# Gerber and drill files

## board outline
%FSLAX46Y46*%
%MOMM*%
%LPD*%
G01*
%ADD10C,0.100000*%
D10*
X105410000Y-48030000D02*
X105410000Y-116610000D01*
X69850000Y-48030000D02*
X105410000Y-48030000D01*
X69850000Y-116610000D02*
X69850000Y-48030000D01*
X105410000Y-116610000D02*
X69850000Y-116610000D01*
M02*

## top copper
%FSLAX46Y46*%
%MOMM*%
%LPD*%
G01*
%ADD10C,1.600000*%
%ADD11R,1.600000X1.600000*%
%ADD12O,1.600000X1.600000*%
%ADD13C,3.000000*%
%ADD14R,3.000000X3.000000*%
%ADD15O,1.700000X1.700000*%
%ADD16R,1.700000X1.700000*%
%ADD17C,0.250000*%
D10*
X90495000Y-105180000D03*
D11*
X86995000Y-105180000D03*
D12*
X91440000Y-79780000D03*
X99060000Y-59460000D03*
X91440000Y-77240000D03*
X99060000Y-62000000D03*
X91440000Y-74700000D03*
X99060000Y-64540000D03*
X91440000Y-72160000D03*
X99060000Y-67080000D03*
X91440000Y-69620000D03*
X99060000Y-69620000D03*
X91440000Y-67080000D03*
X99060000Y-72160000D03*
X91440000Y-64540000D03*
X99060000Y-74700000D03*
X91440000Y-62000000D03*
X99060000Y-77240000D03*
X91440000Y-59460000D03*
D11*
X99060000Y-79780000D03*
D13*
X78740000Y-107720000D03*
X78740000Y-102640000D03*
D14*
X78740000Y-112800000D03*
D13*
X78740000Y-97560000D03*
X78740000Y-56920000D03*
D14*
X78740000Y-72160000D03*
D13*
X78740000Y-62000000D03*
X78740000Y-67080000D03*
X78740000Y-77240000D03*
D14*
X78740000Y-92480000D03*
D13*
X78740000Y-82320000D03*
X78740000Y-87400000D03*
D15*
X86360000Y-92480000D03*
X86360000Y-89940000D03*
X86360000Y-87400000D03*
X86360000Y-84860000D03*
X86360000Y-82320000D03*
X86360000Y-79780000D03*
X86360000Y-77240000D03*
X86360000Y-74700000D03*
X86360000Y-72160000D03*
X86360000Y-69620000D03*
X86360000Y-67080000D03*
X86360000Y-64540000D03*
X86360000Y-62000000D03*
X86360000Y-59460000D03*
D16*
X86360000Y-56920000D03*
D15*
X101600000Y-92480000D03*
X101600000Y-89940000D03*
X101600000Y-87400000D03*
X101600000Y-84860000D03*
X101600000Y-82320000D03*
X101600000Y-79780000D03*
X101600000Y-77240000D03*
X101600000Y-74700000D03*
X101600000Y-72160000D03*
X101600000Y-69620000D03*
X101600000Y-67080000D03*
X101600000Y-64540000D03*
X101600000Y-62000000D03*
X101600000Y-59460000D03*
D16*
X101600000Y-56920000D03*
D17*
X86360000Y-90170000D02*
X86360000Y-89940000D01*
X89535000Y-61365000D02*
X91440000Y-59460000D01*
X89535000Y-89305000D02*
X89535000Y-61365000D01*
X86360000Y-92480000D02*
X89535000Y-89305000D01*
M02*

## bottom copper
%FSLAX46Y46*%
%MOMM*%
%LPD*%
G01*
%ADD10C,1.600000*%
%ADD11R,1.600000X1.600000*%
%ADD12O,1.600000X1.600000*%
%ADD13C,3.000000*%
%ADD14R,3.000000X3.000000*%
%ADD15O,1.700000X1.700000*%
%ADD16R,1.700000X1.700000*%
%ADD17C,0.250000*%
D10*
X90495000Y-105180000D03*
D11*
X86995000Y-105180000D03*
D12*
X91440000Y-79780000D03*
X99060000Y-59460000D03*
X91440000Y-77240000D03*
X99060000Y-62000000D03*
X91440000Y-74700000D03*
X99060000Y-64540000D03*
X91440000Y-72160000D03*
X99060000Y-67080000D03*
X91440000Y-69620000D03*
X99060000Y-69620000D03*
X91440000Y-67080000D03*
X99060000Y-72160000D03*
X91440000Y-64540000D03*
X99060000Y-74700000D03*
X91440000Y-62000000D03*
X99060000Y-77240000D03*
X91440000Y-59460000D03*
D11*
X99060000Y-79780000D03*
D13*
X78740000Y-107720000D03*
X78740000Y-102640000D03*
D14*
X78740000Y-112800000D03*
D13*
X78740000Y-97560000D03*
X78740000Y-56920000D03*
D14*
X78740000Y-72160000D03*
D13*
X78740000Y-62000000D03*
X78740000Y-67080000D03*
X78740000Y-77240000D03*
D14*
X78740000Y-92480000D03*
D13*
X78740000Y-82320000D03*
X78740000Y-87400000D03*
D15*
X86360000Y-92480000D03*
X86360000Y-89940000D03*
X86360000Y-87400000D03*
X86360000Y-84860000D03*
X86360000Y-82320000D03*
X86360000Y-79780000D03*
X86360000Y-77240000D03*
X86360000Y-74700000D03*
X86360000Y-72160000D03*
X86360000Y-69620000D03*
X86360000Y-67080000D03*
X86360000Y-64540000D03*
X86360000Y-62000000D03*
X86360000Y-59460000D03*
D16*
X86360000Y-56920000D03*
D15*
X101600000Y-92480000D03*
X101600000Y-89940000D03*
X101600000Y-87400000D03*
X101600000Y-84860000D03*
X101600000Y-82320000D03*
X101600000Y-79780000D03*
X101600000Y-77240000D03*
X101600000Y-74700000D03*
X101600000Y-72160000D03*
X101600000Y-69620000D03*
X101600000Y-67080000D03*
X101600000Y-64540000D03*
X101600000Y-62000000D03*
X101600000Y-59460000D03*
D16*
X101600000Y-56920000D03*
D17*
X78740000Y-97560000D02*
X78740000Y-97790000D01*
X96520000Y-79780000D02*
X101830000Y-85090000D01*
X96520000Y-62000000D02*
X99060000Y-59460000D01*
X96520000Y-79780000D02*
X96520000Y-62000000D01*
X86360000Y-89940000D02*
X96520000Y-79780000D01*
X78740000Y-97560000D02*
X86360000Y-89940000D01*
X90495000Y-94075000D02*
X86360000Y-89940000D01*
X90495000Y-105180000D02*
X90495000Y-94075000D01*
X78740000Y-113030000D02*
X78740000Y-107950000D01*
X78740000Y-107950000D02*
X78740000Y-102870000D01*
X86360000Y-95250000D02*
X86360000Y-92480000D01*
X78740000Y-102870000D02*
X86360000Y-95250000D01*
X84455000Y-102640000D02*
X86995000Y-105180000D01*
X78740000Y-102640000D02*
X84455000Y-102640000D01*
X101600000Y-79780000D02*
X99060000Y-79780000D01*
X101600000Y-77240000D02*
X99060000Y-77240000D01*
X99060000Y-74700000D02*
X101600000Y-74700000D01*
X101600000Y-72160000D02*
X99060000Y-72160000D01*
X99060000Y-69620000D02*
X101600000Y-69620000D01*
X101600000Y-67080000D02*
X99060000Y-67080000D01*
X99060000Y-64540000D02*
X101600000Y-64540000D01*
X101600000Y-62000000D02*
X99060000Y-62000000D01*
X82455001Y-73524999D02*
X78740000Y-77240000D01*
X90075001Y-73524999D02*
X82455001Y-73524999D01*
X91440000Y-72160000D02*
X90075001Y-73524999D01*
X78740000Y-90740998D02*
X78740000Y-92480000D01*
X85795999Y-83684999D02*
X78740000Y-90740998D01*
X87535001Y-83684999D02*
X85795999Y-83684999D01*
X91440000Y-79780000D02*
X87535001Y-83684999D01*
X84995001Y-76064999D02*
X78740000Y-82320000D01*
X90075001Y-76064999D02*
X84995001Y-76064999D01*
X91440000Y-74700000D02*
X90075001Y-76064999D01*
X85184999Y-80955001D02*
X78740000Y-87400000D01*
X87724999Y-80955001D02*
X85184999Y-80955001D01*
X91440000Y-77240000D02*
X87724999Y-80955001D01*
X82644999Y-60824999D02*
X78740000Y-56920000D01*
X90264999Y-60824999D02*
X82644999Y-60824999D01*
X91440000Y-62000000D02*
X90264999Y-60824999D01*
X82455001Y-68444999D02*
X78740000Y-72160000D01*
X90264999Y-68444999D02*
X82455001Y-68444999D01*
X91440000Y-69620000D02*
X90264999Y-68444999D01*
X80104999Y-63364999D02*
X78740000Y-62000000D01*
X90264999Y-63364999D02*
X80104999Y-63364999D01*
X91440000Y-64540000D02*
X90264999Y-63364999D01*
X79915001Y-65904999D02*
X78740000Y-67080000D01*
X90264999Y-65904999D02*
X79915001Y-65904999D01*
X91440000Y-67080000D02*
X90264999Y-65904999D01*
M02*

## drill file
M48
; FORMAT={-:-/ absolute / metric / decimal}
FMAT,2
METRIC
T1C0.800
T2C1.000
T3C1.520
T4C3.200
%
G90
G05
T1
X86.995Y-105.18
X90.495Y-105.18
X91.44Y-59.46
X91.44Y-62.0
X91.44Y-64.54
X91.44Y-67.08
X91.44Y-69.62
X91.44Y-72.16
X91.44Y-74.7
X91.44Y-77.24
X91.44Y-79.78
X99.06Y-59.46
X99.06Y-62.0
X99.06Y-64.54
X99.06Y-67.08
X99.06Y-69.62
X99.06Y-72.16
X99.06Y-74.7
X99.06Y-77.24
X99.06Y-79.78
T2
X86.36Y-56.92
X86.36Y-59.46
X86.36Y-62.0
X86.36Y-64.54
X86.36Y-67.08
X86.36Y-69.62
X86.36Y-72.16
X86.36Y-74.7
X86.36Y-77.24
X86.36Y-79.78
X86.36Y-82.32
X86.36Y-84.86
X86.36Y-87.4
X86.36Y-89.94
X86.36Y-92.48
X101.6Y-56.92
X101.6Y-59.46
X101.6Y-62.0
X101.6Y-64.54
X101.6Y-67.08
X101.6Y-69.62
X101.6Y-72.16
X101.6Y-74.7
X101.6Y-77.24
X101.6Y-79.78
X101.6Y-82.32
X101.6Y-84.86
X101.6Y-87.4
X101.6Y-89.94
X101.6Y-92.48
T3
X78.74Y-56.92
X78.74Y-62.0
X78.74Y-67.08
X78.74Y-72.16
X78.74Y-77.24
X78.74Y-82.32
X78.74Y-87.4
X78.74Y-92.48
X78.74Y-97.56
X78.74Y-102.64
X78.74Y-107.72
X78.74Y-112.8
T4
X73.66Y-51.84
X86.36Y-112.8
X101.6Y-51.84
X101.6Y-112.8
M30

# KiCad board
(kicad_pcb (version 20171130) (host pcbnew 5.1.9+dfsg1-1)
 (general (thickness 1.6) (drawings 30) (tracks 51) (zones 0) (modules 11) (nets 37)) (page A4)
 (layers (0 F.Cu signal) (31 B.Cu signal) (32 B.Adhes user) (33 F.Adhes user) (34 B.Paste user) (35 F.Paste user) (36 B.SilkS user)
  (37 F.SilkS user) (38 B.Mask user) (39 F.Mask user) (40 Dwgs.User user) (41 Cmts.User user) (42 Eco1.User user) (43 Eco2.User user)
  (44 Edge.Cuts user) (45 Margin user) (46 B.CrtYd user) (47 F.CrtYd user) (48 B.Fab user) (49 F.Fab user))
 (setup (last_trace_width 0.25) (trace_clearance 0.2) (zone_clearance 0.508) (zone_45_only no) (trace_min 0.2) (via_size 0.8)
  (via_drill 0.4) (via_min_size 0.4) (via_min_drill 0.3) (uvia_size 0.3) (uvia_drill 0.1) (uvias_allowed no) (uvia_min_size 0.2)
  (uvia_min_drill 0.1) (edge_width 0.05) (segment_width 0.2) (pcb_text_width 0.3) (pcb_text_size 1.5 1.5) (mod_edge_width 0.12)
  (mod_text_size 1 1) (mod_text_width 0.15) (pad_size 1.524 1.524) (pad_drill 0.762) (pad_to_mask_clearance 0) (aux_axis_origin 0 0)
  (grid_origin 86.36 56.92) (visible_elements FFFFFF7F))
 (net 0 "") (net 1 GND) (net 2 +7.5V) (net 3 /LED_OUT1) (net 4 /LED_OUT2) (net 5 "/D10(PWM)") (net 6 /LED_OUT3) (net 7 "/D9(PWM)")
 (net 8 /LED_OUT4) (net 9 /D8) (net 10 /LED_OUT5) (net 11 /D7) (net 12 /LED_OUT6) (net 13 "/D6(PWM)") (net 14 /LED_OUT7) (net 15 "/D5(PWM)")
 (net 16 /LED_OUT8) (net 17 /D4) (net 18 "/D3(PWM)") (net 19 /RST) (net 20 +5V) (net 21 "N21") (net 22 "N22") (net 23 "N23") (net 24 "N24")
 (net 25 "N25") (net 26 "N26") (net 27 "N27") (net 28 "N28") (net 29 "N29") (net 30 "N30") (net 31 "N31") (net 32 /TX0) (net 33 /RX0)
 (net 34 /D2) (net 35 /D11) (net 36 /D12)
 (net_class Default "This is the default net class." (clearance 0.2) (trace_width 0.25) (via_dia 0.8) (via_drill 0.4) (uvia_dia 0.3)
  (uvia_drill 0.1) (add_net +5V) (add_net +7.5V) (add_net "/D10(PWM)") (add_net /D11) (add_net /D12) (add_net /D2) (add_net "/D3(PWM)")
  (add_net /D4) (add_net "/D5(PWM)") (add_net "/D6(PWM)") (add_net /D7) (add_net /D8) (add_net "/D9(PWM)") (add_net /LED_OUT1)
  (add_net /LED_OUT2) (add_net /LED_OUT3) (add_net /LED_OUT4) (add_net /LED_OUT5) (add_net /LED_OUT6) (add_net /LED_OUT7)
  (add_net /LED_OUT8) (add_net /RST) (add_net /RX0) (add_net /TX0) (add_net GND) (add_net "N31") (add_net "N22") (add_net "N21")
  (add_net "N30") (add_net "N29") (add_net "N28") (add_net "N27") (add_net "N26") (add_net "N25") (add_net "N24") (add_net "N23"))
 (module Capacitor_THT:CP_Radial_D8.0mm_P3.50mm (layer F.Cu) (at 86.995 105.18)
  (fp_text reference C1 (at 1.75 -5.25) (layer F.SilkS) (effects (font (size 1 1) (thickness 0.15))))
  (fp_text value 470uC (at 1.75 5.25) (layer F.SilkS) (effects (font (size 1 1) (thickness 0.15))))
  (pad 2 thru_hole circle (at 3.5 0) (size 1.6 1.6) (drill 0.8) (layers *.Cu *.Mask) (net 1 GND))
  (pad 1 thru_hole rect (at 0 0) (size 1.6 1.6) (drill 0.8) (layers *.Cu *.Mask) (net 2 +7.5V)))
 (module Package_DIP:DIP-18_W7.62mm (layer F.Cu) (at 99.06 79.78 180)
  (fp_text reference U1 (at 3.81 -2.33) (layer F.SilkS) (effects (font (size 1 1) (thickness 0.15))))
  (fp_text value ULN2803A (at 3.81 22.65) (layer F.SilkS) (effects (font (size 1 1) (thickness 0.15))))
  (pad 18 thru_hole oval (at 7.62 0 180) (size 1.6 1.6) (drill 0.8) (layers *.Cu *.Mask) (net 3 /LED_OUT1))
  (pad 9 thru_hole oval (at 0 20.32 180) (size 1.6 1.6) (drill 0.8) (layers *.Cu *.Mask) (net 1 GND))
  (pad 17 thru_hole oval (at 7.62 2.54 180) (size 1.6 1.6) (drill 0.8) (layers *.Cu *.Mask) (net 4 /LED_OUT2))
  (pad 8 thru_hole oval (at 0 17.78 180) (size 1.6 1.6) (drill 0.8) (layers *.Cu *.Mask) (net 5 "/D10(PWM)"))
  (pad 16 thru_hole oval (at 7.62 5.08 180) (size 1.6 1.6) (drill 0.8) (layers *.Cu *.Mask) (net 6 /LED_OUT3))
  (pad 7 thru_hole oval (at 0 15.24 180) (size 1.6 1.6) (drill 0.8) (layers *.Cu *.Mask) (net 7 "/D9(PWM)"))
  (pad 15 thru_hole oval (at 7.62 7.62 180) (size 1.6 1.6) (drill 0.8) (layers *.Cu *.Mask) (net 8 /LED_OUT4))
  (pad 6 thru_hole oval (at 0 12.7 180) (size 1.6 1.6) (drill 0.8) (layers *.Cu *.Mask) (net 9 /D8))
  (pad 14 thru_hole oval (at 7.62 10.16 180) (size 1.6 1.6) (drill 0.8) (layers *.Cu *.Mask) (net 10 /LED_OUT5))
  (pad 5 thru_hole oval (at 0 10.16 180) (size 1.6 1.6) (drill 0.8) (layers *.Cu *.Mask) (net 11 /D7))
  (pad 13 thru_hole oval (at 7.62 12.7 180) (size 1.6 1.6) (drill 0.8) (layers *.Cu *.Mask) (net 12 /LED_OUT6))
  (pad 4 thru_hole oval (at 0 7.62 180) (size 1.6 1.6) (drill 0.8) (layers *.Cu *.Mask) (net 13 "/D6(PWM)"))
  (pad 12 thru_hole oval (at 7.62 15.24 180) (size 1.6 1.6) (drill 0.8) (layers *.Cu *.Mask) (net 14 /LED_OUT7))
  (pad 3 thru_hole oval (at 0 5.08 180) (size 1.6 1.6) (drill 0.8) (layers *.Cu *.Mask) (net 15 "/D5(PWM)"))
  (pad 11 thru_hole oval (at 7.62 17.78 180) (size 1.6 1.6) (drill 0.8) (layers *.Cu *.Mask) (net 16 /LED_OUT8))
  (pad 2 thru_hole oval (at 0 2.54 180) (size 1.6 1.6) (drill 0.8) (layers *.Cu *.Mask) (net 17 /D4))
  (pad 10 thru_hole oval (at 7.62 20.32 180) (size 1.6 1.6) (drill 0.8) (layers *.Cu *.Mask) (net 2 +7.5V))
  (pad 1 thru_hole rect (at 0 0 180) (size 1.6 1.6) (drill 0.8) (layers *.Cu *.Mask) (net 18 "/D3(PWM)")))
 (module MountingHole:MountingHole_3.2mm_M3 (layer F.Cu) (at 101.6 51.84)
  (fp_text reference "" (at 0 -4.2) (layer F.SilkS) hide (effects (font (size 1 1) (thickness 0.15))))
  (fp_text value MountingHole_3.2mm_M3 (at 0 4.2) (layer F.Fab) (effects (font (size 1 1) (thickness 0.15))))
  (pad 1 np_thru_hole circle (at 0 0) (size 3.2 3.2) (drill 3.2) (layers *.Cu *.Mask)))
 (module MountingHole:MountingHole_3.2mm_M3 (layer F.Cu) (at 73.66 51.84)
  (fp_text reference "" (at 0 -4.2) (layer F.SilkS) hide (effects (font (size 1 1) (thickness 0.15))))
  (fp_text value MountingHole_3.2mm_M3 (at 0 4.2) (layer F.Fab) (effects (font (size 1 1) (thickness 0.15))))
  (pad 1 np_thru_hole circle (at 0 0) (size 3.2 3.2) (drill 3.2) (layers *.Cu *.Mask)))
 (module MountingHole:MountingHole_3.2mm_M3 (layer F.Cu) (at 101.6 112.8)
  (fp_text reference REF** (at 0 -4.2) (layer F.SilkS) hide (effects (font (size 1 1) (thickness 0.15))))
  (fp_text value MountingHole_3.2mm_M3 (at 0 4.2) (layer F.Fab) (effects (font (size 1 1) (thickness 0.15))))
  (pad 1 np_thru_hole circle (at 0 0) (size 3.2 3.2) (drill 3.2) (layers *.Cu *.Mask)))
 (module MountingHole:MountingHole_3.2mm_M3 (layer F.Cu) (at 86.36 112.8)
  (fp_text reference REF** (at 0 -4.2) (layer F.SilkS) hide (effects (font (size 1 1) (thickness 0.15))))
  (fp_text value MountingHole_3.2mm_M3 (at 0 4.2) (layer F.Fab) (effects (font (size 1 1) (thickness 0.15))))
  (pad 1 np_thru_hole circle (at 0 0) (size 3.2 3.2) (drill 3.2) (layers *.Cu *.Mask)))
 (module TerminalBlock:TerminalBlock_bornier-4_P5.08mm (layer F.Cu) (at 78.74 112.8 90)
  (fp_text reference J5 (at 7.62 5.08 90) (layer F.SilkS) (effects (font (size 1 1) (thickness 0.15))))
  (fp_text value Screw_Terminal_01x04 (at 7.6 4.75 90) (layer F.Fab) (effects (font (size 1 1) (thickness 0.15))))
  (pad 2 thru_hole circle (at 5.08 0 90) (size 3 3) (drill 1.52) (layers *.Cu *.Mask) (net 2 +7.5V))
  (pad 3 thru_hole circle (at 10.16 0 90) (size 3 3) (drill 1.52) (layers *.Cu *.Mask) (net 2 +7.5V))
  (pad 1 thru_hole rect (at 0 0 90) (size 3 3) (drill 1.52) (layers *.Cu *.Mask) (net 2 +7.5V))
  (pad 4 thru_hole circle (at 15.24 0 90) (size 3 3) (drill 1.52) (layers *.Cu *.Mask) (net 1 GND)))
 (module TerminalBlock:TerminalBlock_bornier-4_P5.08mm (layer F.Cu) (at 78.74 72.16 90)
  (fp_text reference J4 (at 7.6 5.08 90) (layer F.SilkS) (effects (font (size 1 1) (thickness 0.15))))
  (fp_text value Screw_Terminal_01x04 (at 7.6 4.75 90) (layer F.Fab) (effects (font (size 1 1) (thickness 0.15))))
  (pad 4 thru_hole circle (at 15.24 0 90) (size 3 3) (drill 1.52) (layers *.Cu *.Mask) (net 16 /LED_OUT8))
  (pad 1 thru_hole rect (at 0 0 90) (size 3 3) (drill 1.52) (layers *.Cu *.Mask) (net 10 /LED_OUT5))
  (pad 3 thru_hole circle (at 10.16 0 90) (size 3 3) (drill 1.52) (layers *.Cu *.Mask) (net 14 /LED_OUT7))
  (pad 2 thru_hole circle (at 5.08 0 90) (size 3 3) (drill 1.52) (layers *.Cu *.Mask) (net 12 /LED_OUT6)))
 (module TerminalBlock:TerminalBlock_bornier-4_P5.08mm (layer F.Cu) (at 78.74 92.48 90)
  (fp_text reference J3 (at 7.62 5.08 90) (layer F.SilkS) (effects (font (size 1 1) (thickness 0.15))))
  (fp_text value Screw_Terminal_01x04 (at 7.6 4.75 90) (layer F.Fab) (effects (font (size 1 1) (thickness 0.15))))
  (pad 4 thru_hole circle (at 15.24 0 90) (size 3 3) (drill 1.52) (layers *.Cu *.Mask) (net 8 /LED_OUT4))
  (pad 1 thru_hole rect (at 0 0 90) (size 3 3) (drill 1.52) (layers *.Cu *.Mask) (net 3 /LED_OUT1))
  (pad 3 thru_hole circle (at 10.16 0 90) (size 3 3) (drill 1.52) (layers *.Cu *.Mask) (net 6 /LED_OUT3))
  (pad 2 thru_hole circle (at 5.08 0 90) (size 3 3) (drill 1.52) (layers *.Cu *.Mask) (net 4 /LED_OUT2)))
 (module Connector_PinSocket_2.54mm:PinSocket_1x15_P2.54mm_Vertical (layer F.Cu) (at 86.36 56.92)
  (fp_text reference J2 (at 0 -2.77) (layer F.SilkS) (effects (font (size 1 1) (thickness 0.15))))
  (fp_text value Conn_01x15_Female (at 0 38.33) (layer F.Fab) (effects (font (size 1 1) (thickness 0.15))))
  (pad 15 thru_hole oval (at 0 35.56) (size 1.7 1.7) (drill 1) (layers *.Cu *.Mask) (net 2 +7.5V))
  (pad 14 thru_hole oval (at 0 33.02) (size 1.7 1.7) (drill 1) (layers *.Cu *.Mask) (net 1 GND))
  (pad 13 thru_hole oval (at 0 30.48) (size 1.7 1.7) (drill 1) (layers *.Cu *.Mask) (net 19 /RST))
  (pad 12 thru_hole oval (at 0 27.94) (size 1.7 1.7) (drill 1) (layers *.Cu *.Mask) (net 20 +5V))
  (pad 11 thru_hole oval (at 0 25.4) (size 1.7 1.7) (drill 1) (layers *.Cu *.Mask) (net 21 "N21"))
  (pad 10 thru_hole oval (at 0 22.86) (size 1.7 1.7) (drill 1) (layers *.Cu *.Mask) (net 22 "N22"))
  (pad 9 thru_hole oval (at 0 20.32) (size 1.7 1.7) (drill 1) (layers *.Cu *.Mask) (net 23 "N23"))
  (pad 8 thru_hole oval (at 0 17.78) (size 1.7 1.7) (drill 1) (layers *.Cu *.Mask) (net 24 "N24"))
  (pad 7 thru_hole oval (at 0 15.24) (size 1.7 1.7) (drill 1) (layers *.Cu *.Mask) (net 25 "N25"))
  (pad 6 thru_hole oval (at 0 12.7) (size 1.7 1.7) (drill 1) (layers *.Cu *.Mask) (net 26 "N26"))
  (pad 5 thru_hole oval (at 0 10.16) (size 1.7 1.7) (drill 1) (layers *.Cu *.Mask) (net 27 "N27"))
  (pad 4 thru_hole oval (at 0 7.62) (size 1.7 1.7) (drill 1) (layers *.Cu *.Mask) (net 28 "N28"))
  (pad 3 thru_hole oval (at 0 5.08) (size 1.7 1.7) (drill 1) (layers *.Cu *.Mask) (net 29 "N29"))
  (pad 2 thru_hole oval (at 0 2.54) (size 1.7 1.7) (drill 1) (layers *.Cu *.Mask) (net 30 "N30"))
  (pad 1 thru_hole rect (at 0 0) (size 1.7 1.7) (drill 1) (layers *.Cu *.Mask) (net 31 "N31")))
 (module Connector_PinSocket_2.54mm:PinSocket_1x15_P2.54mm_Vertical (layer F.Cu) (at 101.6 56.92)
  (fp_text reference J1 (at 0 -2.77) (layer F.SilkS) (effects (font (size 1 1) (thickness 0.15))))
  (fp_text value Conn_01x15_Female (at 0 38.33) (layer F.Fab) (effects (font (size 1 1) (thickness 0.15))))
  (pad 15 thru_hole oval (at 0 35.56) (size 1.7 1.7) (drill 1) (layers *.Cu *.Mask) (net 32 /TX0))
  (pad 14 thru_hole oval (at 0 33.02) (size 1.7 1.7) (drill 1) (layers *.Cu *.Mask) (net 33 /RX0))
  (pad 13 thru_hole oval (at 0 30.48) (size 1.7 1.7) (drill 1) (layers *.Cu *.Mask) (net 19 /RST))
  (pad 12 thru_hole oval (at 0 27.94) (size 1.7 1.7) (drill 1) (layers *.Cu *.Mask) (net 1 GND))
  (pad 11 thru_hole oval (at 0 25.4) (size 1.7 1.7) (drill 1) (layers *.Cu *.Mask) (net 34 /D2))
  (pad 10 thru_hole oval (at 0 22.86) (size 1.7 1.7) (drill 1) (layers *.Cu *.Mask) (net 18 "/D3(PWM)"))
  (pad 9 thru_hole oval (at 0 20.32) (size 1.7 1.7) (drill 1) (layers *.Cu *.Mask) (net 17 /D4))
  (pad 8 thru_hole oval (at 0 17.78) (size 1.7 1.7) (drill 1) (layers *.Cu *.Mask) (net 15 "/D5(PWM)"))
  (pad 7 thru_hole oval (at 0 15.24) (size 1.7 1.7) (drill 1) (layers *.Cu *.Mask) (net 13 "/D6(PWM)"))
  (pad 6 thru_hole oval (at 0 12.7) (size 1.7 1.7) (drill 1) (layers *.Cu *.Mask) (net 11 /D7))
  (pad 5 thru_hole oval (at 0 10.16) (size 1.7 1.7) (drill 1) (layers *.Cu *.Mask) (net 9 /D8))
  (pad 4 thru_hole oval (at 0 7.62) (size 1.7 1.7) (drill 1) (layers *.Cu *.Mask) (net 7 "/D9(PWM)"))
  (pad 3 thru_hole oval (at 0 5.08) (size 1.7 1.7) (drill 1) (layers *.Cu *.Mask) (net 5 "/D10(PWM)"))
  (pad 2 thru_hole oval (at 0 2.54) (size 1.7 1.7) (drill 1) (layers *.Cu *.Mask) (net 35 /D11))
  (pad 1 thru_hole rect (at 0 0) (size 1.7 1.7) (drill 1) (layers *.Cu *.Mask) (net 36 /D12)))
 (gr_line (start 105.41 48.03) (end 105.41 116.61) (layer Edge.Cuts) (width 0.1))
 (gr_line (start 69.85 48.03) (end 105.41 48.03) (layer Edge.Cuts) (width 0.1))
 (gr_line (start 69.85 116.61) (end 69.85 48.03) (layer Edge.Cuts) (width 0.1))
 (gr_line (start 105.41 116.61) (end 69.85 116.61) (layer Edge.Cuts) (width 0.1))
 (segment (start 86.36 90.17) (end 86.36 89.94) (width 0.25) (layer F.Cu) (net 1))
 (segment (start 78.74 97.56) (end 78.74 97.79) (width 0.25) (layer B.Cu) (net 1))
 (segment (start 96.52 79.78) (end 101.83 85.09) (width 0.25) (layer B.Cu) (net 1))
 (segment (start 96.52 62) (end 99.06 59.46) (width 0.25) (layer B.Cu) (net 1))
 (segment (start 96.52 79.78) (end 96.52 62) (width 0.25) (layer B.Cu) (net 1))
 (segment (start 86.36 89.94) (end 96.52 79.78) (width 0.25) (layer B.Cu) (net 1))
 (segment (start 78.74 97.56) (end 86.36 89.94) (width 0.25) (layer B.Cu) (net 1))
 (segment (start 90.495 94.075) (end 86.36 89.94) (width 0.25) (layer B.Cu) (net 1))
 (segment (start 90.495 105.18) (end 90.495 94.075) (width 0.25) (layer B.Cu) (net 1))
 (segment (start 78.74 113.03) (end 78.74 107.95) (width 0.25) (layer B.Cu) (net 2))
 (segment (start 78.74 107.95) (end 78.74 102.87) (width 0.25) (layer B.Cu) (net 2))
 (segment (start 86.36 95.25) (end 86.36 92.48) (width 0.25) (layer B.Cu) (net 2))
 (segment (start 78.74 102.87) (end 86.36 95.25) (width 0.25) (layer B.Cu) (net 2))
 (segment (start 89.535 61.365) (end 91.44 59.46) (width 0.25) (layer F.Cu) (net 2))
 (segment (start 89.535 89.305) (end 89.535 61.365) (width 0.25) (layer F.Cu) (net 2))
 (segment (start 86.36 92.48) (end 89.535 89.305) (width 0.25) (layer F.Cu) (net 2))
 (segment (start 84.455 102.64) (end 86.995 105.18) (width 0.25) (layer B.Cu) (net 2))
 (segment (start 78.74 102.64) (end 84.455 102.64) (width 0.25) (layer B.Cu) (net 2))
 (segment (start 101.6 79.78) (end 99.06 79.78) (width 0.25) (layer B.Cu) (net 18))
 (segment (start 101.6 77.24) (end 99.06 77.24) (width 0.25) (layer B.Cu) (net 17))
 (segment (start 99.06 74.7) (end 101.6 74.7) (width 0.25) (layer B.Cu) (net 15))
 (segment (start 101.6 72.16) (end 99.06 72.16) (width 0.25) (layer B.Cu) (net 13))
 (segment (start 99.06 69.62) (end 101.6 69.62) (width 0.25) (layer B.Cu) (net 11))
 (segment (start 101.6 67.08) (end 99.06 67.08) (width 0.25) (layer B.Cu) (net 9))
 (segment (start 99.06 64.54) (end 101.6 64.54) (width 0.25) (layer B.Cu) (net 7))
 (segment (start 101.6 62) (end 99.06 62) (width 0.25) (layer B.Cu) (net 5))
 (segment (start 82.455001 73.524999) (end 78.74 77.24) (width 0.25) (layer B.Cu) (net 8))
 (segment (start 90.075001 73.524999) (end 82.455001 73.524999) (width 0.25) (layer B.Cu) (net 8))
 (segment (start 91.44 72.16) (end 90.075001 73.524999) (width 0.25) (layer B.Cu) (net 8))
 (segment (start 78.74 90.740998) (end 78.74 92.48) (width 0.25) (layer B.Cu) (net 3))
 (segment (start 85.795999 83.684999) (end 78.74 90.740998) (width 0.25) (layer B.Cu) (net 3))
 (segment (start 87.535001 83.684999) (end 85.795999 83.684999) (width 0.25) (layer B.Cu) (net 3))
 (segment (start 91.44 79.78) (end 87.535001 83.684999) (width 0.25) (layer B.Cu) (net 3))
 (segment (start 84.995001 76.064999) (end 78.74 82.32) (width 0.25) (layer B.Cu) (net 6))
 (segment (start 90.075001 76.064999) (end 84.995001 76.064999) (width 0.25) (layer B.Cu) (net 6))
 (segment (start 91.44 74.7) (end 90.075001 76.064999) (width 0.25) (layer B.Cu) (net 6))
 (segment (start 85.184999 80.955001) (end 78.74 87.4) (width 0.25) (layer B.Cu) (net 4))
 (segment (start 87.724999 80.955001) (end 85.184999 80.955001) (width 0.25) (layer B.Cu) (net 4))
 (segment (start 91.44 77.24) (end 87.724999 80.955001) (width 0.25) (layer B.Cu) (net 4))
 (segment (start 82.644999 60.824999) (end 78.74 56.92) (width 0.25) (layer B.Cu) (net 16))
 (segment (start 90.264999 60.824999) (end 82.644999 60.824999) (width 0.25) (layer B.Cu) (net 16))
 (segment (start 91.44 62) (end 90.264999 60.824999) (width 0.25) (layer B.Cu) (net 16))
 (segment (start 82.455001 68.444999) (end 78.74 72.16) (width 0.25) (layer B.Cu) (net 10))
 (segment (start 90.264999 68.444999) (end 82.455001 68.444999) (width 0.25) (layer B.Cu) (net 10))
 (segment (start 91.44 69.62) (end 90.264999 68.444999) (width 0.25) (layer B.Cu) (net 10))
 (segment (start 80.104999 63.364999) (end 78.74 62) (width 0.25) (layer B.Cu) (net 14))
 (segment (start 90.264999 63.364999) (end 80.104999 63.364999) (width 0.25) (layer B.Cu) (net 14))
 (segment (start 91.44 64.54) (end 90.264999 63.364999) (width 0.25) (layer B.Cu) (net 14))
 (segment (start 79.915001 65.904999) (end 78.74 67.08) (width 0.25) (layer B.Cu) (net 12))
 (segment (start 90.264999 65.904999) (end 79.915001 65.904999) (width 0.25) (layer B.Cu) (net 12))
 (segment (start 91.44 67.08) (end 90.264999 65.904999) (width 0.25) (layer B.Cu) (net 12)))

